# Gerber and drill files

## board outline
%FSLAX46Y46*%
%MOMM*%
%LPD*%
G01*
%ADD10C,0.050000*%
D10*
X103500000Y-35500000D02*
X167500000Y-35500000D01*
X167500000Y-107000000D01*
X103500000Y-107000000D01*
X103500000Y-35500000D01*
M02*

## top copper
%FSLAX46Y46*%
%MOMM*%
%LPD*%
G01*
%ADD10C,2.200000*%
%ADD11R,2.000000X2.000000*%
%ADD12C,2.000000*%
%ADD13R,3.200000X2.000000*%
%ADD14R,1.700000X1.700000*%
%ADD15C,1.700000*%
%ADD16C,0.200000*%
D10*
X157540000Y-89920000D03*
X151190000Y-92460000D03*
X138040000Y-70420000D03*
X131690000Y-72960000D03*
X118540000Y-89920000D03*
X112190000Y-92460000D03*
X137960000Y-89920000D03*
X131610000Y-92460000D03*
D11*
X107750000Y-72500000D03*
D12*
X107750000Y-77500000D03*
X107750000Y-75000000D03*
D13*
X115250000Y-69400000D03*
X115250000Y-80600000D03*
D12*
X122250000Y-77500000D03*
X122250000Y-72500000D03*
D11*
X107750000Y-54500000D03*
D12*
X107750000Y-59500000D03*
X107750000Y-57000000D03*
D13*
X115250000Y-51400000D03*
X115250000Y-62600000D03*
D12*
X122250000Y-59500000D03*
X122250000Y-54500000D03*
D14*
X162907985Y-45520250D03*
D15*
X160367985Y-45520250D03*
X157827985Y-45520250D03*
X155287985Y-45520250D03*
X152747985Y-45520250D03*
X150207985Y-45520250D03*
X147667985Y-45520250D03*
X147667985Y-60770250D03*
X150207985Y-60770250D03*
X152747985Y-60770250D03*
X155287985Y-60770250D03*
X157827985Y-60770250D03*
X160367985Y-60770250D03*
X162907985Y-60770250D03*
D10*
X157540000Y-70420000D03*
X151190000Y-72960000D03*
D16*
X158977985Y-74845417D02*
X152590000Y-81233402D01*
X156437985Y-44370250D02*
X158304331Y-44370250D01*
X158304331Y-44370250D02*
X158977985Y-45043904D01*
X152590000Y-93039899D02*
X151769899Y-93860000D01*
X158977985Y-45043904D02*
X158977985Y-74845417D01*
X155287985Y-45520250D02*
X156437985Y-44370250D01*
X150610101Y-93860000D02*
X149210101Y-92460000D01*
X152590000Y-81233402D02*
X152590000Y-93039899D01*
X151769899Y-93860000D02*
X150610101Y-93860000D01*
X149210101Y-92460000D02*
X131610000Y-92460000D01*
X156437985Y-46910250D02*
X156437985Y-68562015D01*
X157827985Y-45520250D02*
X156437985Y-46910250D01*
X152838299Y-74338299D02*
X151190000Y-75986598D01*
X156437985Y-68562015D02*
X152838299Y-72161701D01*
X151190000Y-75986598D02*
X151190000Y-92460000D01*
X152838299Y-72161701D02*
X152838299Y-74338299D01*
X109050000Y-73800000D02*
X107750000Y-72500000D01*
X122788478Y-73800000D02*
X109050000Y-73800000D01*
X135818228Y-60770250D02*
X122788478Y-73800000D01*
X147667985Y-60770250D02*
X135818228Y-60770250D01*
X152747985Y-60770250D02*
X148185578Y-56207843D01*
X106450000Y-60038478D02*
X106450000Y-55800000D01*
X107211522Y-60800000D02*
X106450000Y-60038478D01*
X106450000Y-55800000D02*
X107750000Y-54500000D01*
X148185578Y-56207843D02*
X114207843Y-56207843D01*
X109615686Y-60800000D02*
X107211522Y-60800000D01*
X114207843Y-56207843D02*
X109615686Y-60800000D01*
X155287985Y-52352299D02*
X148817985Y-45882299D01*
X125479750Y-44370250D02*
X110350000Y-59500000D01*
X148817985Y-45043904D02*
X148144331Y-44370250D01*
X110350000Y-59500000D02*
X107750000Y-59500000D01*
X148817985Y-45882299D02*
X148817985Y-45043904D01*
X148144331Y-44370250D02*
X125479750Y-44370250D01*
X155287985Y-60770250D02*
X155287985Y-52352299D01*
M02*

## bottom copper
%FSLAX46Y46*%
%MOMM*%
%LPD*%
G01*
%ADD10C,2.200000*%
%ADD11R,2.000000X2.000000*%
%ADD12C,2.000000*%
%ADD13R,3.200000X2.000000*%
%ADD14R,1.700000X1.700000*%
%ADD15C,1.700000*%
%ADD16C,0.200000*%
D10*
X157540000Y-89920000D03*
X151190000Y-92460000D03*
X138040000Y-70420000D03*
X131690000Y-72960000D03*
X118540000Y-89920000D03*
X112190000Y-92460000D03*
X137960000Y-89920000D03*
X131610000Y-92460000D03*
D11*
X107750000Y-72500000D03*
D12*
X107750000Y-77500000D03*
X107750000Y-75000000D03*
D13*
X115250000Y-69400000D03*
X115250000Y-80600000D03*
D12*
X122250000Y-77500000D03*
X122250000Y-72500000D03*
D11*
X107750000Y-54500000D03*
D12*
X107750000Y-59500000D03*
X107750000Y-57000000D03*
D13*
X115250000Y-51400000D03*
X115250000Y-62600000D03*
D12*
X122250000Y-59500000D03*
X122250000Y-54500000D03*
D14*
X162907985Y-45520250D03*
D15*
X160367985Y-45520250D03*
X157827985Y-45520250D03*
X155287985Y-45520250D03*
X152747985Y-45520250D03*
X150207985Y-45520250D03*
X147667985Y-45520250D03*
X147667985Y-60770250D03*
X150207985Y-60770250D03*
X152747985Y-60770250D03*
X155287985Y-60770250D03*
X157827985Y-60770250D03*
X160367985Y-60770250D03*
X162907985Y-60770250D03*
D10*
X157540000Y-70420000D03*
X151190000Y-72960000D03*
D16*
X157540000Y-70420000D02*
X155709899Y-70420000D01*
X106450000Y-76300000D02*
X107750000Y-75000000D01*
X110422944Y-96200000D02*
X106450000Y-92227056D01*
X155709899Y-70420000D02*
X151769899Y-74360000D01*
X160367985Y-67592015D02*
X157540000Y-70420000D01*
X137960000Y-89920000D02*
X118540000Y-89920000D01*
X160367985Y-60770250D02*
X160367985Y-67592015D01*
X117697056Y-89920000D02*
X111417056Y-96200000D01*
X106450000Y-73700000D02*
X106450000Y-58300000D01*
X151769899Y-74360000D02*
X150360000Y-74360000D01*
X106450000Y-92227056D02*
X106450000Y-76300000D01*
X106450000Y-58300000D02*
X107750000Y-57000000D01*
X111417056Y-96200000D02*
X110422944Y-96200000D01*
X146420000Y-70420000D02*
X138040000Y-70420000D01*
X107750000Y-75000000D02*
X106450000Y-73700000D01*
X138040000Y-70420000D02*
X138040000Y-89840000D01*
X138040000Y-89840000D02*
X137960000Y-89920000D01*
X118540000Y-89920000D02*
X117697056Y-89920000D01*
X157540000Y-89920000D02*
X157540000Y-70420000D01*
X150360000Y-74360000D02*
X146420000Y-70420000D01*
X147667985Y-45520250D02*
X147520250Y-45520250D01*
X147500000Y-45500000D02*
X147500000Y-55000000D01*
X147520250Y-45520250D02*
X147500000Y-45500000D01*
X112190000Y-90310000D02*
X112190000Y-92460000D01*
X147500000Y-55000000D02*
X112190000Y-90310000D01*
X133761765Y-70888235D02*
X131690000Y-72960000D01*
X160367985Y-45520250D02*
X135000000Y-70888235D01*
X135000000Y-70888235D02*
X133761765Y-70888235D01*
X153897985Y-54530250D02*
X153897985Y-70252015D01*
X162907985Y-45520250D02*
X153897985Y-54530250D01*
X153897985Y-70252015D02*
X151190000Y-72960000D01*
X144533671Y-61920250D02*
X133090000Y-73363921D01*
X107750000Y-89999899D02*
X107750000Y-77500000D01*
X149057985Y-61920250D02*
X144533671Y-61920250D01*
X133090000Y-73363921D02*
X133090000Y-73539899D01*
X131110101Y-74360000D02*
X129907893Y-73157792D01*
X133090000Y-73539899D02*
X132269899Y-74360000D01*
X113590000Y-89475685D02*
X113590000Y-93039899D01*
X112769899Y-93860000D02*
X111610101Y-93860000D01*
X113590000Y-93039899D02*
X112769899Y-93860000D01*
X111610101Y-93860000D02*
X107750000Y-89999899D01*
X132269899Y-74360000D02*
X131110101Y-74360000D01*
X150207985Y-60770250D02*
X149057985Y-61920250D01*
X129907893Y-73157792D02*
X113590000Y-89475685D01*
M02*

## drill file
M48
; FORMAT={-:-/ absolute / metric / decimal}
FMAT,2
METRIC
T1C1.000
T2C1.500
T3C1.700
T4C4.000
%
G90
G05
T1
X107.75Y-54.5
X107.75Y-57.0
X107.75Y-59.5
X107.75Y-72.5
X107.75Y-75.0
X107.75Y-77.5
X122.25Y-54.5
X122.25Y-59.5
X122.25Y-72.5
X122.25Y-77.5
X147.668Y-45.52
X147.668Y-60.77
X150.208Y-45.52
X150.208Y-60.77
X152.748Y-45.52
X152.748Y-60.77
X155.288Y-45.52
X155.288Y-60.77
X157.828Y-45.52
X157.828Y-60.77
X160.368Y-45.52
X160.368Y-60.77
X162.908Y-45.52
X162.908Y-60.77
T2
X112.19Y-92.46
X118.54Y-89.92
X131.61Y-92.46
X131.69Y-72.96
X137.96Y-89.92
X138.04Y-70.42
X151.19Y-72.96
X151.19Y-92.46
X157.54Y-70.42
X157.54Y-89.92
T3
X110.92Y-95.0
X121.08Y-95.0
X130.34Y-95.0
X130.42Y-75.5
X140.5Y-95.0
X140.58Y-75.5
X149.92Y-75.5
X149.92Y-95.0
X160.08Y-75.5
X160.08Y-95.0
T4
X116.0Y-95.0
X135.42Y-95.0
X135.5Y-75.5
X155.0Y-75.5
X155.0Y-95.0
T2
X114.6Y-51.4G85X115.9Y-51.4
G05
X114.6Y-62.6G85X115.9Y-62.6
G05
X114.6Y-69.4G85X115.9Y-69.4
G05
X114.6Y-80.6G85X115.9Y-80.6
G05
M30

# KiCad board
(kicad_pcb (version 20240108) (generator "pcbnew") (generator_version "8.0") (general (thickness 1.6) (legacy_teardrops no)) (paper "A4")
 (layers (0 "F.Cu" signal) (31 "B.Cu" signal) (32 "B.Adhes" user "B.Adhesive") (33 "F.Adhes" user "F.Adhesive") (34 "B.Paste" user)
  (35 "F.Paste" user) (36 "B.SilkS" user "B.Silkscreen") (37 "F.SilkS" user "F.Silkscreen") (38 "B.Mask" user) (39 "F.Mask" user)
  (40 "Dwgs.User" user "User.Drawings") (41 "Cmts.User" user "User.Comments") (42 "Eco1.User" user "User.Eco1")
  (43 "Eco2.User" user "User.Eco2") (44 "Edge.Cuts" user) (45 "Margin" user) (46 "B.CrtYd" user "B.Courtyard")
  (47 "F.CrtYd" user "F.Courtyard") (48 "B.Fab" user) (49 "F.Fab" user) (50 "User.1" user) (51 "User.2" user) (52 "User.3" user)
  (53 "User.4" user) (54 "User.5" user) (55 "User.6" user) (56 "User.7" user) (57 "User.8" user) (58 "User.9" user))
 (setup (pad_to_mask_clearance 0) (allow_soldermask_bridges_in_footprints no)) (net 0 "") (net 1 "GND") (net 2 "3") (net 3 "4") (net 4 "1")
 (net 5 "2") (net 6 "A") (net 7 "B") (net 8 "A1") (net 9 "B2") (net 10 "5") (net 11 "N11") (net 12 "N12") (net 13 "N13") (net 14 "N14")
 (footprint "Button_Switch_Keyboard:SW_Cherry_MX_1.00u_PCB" (layer "F.Cu") (at 157.54 89.92)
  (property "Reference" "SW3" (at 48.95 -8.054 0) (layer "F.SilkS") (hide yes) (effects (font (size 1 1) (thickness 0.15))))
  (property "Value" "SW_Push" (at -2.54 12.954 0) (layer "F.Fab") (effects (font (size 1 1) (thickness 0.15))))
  (pad "" np_thru_hole circle (at -7.62 5.08) (size 1.7 1.7) (drill 1.7) (layers "*.Cu" "*.Mask"))
  (pad "" np_thru_hole circle (at -2.54 5.08) (size 4 4) (drill 4) (layers "*.Cu" "*.Mask"))
  (pad "" np_thru_hole circle (at 2.54 5.08) (size 1.7 1.7) (drill 1.7) (layers "*.Cu" "*.Mask"))
  (pad "1" thru_hole circle (at 0 0) (size 2.2 2.2) (drill 1.5) (layers "*.Cu" "*.Mask") (remove_unused_layers no) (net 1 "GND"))
  (pad "2" thru_hole circle (at -6.35 2.54) (size 2.2 2.2) (drill 1.5) (layers "*.Cu" "*.Mask") (remove_unused_layers no) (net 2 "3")))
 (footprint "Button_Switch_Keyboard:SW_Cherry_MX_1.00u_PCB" (layer "F.Cu") (at 138.04 70.42)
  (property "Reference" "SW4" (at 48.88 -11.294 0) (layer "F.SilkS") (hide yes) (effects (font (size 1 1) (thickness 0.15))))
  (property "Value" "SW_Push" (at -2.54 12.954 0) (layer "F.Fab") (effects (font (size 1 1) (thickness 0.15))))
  (pad "" np_thru_hole circle (at -7.62 5.08) (size 1.7 1.7) (drill 1.7) (layers "*.Cu" "*.Mask"))
  (pad "" np_thru_hole circle (at -2.54 5.08) (size 4 4) (drill 4) (layers "*.Cu" "*.Mask"))
  (pad "" np_thru_hole circle (at 2.54 5.08) (size 1.7 1.7) (drill 1.7) (layers "*.Cu" "*.Mask"))
  (pad "1" thru_hole circle (at 0 0) (size 2.2 2.2) (drill 1.5) (layers "*.Cu" "*.Mask") (remove_unused_layers no) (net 1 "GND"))
  (pad "2" thru_hole circle (at -6.35 2.54) (size 2.2 2.2) (drill 1.5) (layers "*.Cu" "*.Mask") (remove_unused_layers no) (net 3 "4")))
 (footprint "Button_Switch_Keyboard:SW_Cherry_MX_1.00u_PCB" (layer "F.Cu") (at 118.54 89.92)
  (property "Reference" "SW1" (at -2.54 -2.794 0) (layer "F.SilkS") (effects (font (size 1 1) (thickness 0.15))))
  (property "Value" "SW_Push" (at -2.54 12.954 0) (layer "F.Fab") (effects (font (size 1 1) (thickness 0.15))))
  (pad "" np_thru_hole circle (at -7.62 5.08) (size 1.7 1.7) (drill 1.7) (layers "*.Cu" "*.Mask"))
  (pad "" np_thru_hole circle (at -2.54 5.08) (size 4 4) (drill 4) (layers "*.Cu" "*.Mask"))
  (pad "" np_thru_hole circle (at 2.54 5.08) (size 1.7 1.7) (drill 1.7) (layers "*.Cu" "*.Mask"))
  (pad "1" thru_hole circle (at 0 0) (size 2.2 2.2) (drill 1.5) (layers "*.Cu" "*.Mask") (remove_unused_layers no) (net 1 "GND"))
  (pad "2" thru_hole circle (at -6.35 2.54) (size 2.2 2.2) (drill 1.5) (layers "*.Cu" "*.Mask") (remove_unused_layers no) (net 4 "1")))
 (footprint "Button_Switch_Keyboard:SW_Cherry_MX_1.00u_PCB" (layer "F.Cu") (at 137.96 89.92)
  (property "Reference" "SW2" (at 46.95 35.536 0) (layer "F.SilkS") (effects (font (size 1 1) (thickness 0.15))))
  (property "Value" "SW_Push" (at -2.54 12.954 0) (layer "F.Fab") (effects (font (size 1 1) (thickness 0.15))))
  (pad "" np_thru_hole circle (at -7.62 5.08) (size 1.7 1.7) (drill 1.7) (layers "*.Cu" "*.Mask"))
  (pad "" np_thru_hole circle (at -2.54 5.08) (size 4 4) (drill 4) (layers "*.Cu" "*.Mask"))
  (pad "" np_thru_hole circle (at 2.54 5.08) (size 1.7 1.7) (drill 1.7) (layers "*.Cu" "*.Mask"))
  (pad "1" thru_hole circle (at 0 0) (size 2.2 2.2) (drill 1.5) (layers "*.Cu" "*.Mask") (remove_unused_layers no) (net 1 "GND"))
  (pad "2" thru_hole circle (at -6.35 2.54) (size 2.2 2.2) (drill 1.5) (layers "*.Cu" "*.Mask") (remove_unused_layers no) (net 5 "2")))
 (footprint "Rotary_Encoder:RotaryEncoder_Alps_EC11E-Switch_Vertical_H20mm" (layer "F.Cu") (at 107.75 72.5)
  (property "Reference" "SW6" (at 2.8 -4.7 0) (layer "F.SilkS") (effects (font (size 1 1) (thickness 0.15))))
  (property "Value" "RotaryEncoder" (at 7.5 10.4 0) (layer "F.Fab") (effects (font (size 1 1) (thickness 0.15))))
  (pad "A" thru_hole rect (at 0 0) (size 2 2) (drill 1) (layers "*.Cu" "*.Mask") (remove_unused_layers no) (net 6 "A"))
  (pad "B" thru_hole circle (at 0 5) (size 2 2) (drill 1) (layers "*.Cu" "*.Mask") (remove_unused_layers no) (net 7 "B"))
  (pad "C" thru_hole circle (at 0 2.5) (size 2 2) (drill 1) (layers "*.Cu" "*.Mask") (remove_unused_layers no) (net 1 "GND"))
  (pad "MP" thru_hole rect (at 7.5 -3.1) (size 3.2 2) (drill oval 2.8 1.5) (layers "*.Cu" "*.Mask") (remove_unused_layers no))
  (pad "MP" thru_hole rect (at 7.5 8.1) (size 3.2 2) (drill oval 2.8 1.5) (layers "*.Cu" "*.Mask") (remove_unused_layers no))
  (pad "S1" thru_hole circle (at 14.5 5) (size 2 2) (drill 1) (layers "*.Cu" "*.Mask") (remove_unused_layers no))
  (pad "S2" thru_hole circle (at 14.5 0) (size 2 2) (drill 1) (layers "*.Cu" "*.Mask") (remove_unused_layers no)))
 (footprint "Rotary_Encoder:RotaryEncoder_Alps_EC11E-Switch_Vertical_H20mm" (layer "F.Cu") (at 107.75 54.5)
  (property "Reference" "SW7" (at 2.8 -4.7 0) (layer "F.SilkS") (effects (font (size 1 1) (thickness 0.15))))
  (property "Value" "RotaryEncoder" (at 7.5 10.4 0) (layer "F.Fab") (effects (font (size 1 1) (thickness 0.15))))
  (pad "A" thru_hole rect (at 0 0) (size 2 2) (drill 1) (layers "*.Cu" "*.Mask") (remove_unused_layers no) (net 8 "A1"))
  (pad "B" thru_hole circle (at 0 5) (size 2 2) (drill 1) (layers "*.Cu" "*.Mask") (remove_unused_layers no) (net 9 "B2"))
  (pad "C" thru_hole circle (at 0 2.5) (size 2 2) (drill 1) (layers "*.Cu" "*.Mask") (remove_unused_layers no) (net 1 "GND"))
  (pad "MP" thru_hole rect (at 7.5 -3.1) (size 3.2 2) (drill oval 2.8 1.5) (layers "*.Cu" "*.Mask") (remove_unused_layers no))
  (pad "MP" thru_hole rect (at 7.5 8.1) (size 3.2 2) (drill oval 2.8 1.5) (layers "*.Cu" "*.Mask") (remove_unused_layers no))
  (pad "S1" thru_hole circle (at 14.5 5) (size 2 2) (drill 1) (layers "*.Cu" "*.Mask") (remove_unused_layers no))
  (pad "S2" thru_hole circle (at 14.5 0) (size 2 2) (drill 1) (layers "*.Cu" "*.Mask") (remove_unused_layers no)))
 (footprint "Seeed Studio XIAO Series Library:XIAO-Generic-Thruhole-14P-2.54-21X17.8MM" (layer "F.Cu") (at 155.287985 53.14525 -90)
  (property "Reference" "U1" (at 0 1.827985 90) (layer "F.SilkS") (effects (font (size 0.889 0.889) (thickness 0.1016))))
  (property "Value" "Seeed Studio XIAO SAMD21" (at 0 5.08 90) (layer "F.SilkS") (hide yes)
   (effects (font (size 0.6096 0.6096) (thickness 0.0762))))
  (pad "1" thru_hole rect (at -7.625 -7.62 270) (size 1.7 1.7) (drill 1) (layers "*.Cu" "*.Mask") (remove_unused_layers no) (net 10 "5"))
  (pad "2" thru_hole circle (at -7.625 -5.08 270) (size 1.7 1.7) (drill 1) (layers "*.Cu" "*.Mask") (remove_unused_layers no) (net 3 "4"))
  (pad "3" thru_hole circle (at -7.625 -2.54 270) (size 1.7 1.7) (drill 1) (layers "*.Cu" "*.Mask") (remove_unused_layers no) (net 2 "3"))
  (pad "4" thru_hole circle (at -7.625 0 270) (size 1.7 1.7) (drill 1) (layers "*.Cu" "*.Mask") (remove_unused_layers no) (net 5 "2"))
  (pad "5" thru_hole circle (at -7.625 2.54 270) (size 1.7 1.7) (drill 1) (layers "*.Cu" "*.Mask") (remove_unused_layers no) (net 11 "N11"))
  (pad "6" thru_hole circle (at -7.625 5.08 90) (size 1.7 1.7) (drill 1) (layers "*.Cu" "*.Mask") (remove_unused_layers no) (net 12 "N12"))
  (pad "7" thru_hole circle (at -7.625 7.62 270) (size 1.7 1.7) (drill 1) (layers "*.Cu" "*.Mask") (remove_unused_layers no) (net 4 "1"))
  (pad "8" thru_hole circle (at 7.625 7.62 270) (size 1.7 1.7) (drill 1) (layers "*.Cu" "*.Mask") (remove_unused_layers no) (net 6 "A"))
  (pad "9" thru_hole circle (at 7.625 5.08 270) (size 1.7 1.7) (drill 1) (layers "*.Cu" "*.Mask") (remove_unused_layers no) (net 7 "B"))
  (pad "10" thru_hole circle (at 7.625 2.54 270) (size 1.7 1.7) (drill 1) (layers "*.Cu" "*.Mask") (remove_unused_layers no) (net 8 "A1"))
  (pad "11" thru_hole circle (at 7.625 0 270) (size 1.7 1.7) (drill 1) (layers "*.Cu" "*.Mask") (remove_unused_layers no) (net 9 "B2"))
  (pad "12" thru_hole circle (at 7.625 -2.54 270) (size 1.7 1.7) (drill 1) (layers "*.Cu" "*.Mask") (remove_unused_layers no) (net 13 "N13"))
  (pad "13" thru_hole circle (at 7.625 -5.08 270) (size 1.7 1.7) (drill 1) (layers "*.Cu" "*.Mask") (remove_unused_layers no) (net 1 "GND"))
  (pad "14" thru_hole circle (at 7.625 -7.62 270) (size 1.7 1.7) (drill 1) (layers "*.Cu" "*.Mask") (remove_unused_layers no) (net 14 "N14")))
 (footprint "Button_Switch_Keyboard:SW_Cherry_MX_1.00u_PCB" (layer "F.Cu") (at 157.54 70.42)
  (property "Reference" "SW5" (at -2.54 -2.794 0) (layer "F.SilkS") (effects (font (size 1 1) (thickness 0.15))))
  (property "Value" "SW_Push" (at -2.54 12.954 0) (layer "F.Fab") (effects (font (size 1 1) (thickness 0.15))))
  (pad "" np_thru_hole circle (at -7.62 5.08) (size 1.7 1.7) (drill 1.7) (layers "*.Cu" "*.Mask"))
  (pad "" np_thru_hole circle (at -2.54 5.08) (size 4 4) (drill 4) (layers "*.Cu" "*.Mask"))
  (pad "" np_thru_hole circle (at 2.54 5.08) (size 1.7 1.7) (drill 1.7) (layers "*.Cu" "*.Mask"))
  (pad "1" thru_hole circle (at 0 0) (size 2.2 2.2) (drill 1.5) (layers "*.Cu" "*.Mask") (remove_unused_layers no) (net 1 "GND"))
  (pad "2" thru_hole circle (at -6.35 2.54) (size 2.2 2.2) (drill 1.5) (layers "*.Cu" "*.Mask") (remove_unused_layers no) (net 10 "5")))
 (gr_rect (start 103.5 35.5) (end 167.5 107) (stroke (width 0.05) (type default)) (fill none) (layer "Edge.Cuts"))
 (segment (start 157.54 70.42) (end 155.709899 70.42) (width 0.2) (layer "B.Cu") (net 1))
 (segment (start 106.45 76.3) (end 107.75 75) (width 0.2) (layer "B.Cu") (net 1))
 (segment (start 110.422944 96.2) (end 106.45 92.227056) (width 0.2) (layer "B.Cu") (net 1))
 (segment (start 155.709899 70.42) (end 151.769899 74.36) (width 0.2) (layer "B.Cu") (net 1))
 (segment (start 160.367985 67.592015) (end 157.54 70.42) (width 0.2) (layer "B.Cu") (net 1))
 (segment (start 137.96 89.92) (end 118.54 89.92) (width 0.2) (layer "B.Cu") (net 1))
 (segment (start 160.367985 60.77025) (end 160.367985 67.592015) (width 0.2) (layer "B.Cu") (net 1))
 (segment (start 117.697056 89.92) (end 111.417056 96.2) (width 0.2) (layer "B.Cu") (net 1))
 (segment (start 106.45 73.7) (end 106.45 58.3) (width 0.2) (layer "B.Cu") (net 1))
 (segment (start 151.769899 74.36) (end 150.36 74.36) (width 0.2) (layer "B.Cu") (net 1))
 (segment (start 106.45 92.227056) (end 106.45 76.3) (width 0.2) (layer "B.Cu") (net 1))
 (segment (start 106.45 58.3) (end 107.75 57) (width 0.2) (layer "B.Cu") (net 1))
 (segment (start 111.417056 96.2) (end 110.422944 96.2) (width 0.2) (layer "B.Cu") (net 1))
 (segment (start 146.42 70.42) (end 138.04 70.42) (width 0.2) (layer "B.Cu") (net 1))
 (segment (start 107.75 75) (end 106.45 73.7) (width 0.2) (layer "B.Cu") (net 1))
 (segment (start 138.04 70.42) (end 138.04 89.84) (width 0.2) (layer "B.Cu") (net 1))
 (segment (start 138.04 89.84) (end 137.96 89.92) (width 0.2) (layer "B.Cu") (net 1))
 (segment (start 118.54 89.92) (end 117.697056 89.92) (width 0.2) (layer "B.Cu") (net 1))
 (segment (start 157.54 89.92) (end 157.54 70.42) (width 0.2) (layer "B.Cu") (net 1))
 (segment (start 150.36 74.36) (end 146.42 70.42) (width 0.2) (layer "B.Cu") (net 1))
 (segment (start 147.667985 45.52025) (end 147.52025 45.52025) (width 0.2) (layer "B.Cu") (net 4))
 (segment (start 147.5 45.5) (end 147.5 55) (width 0.2) (layer "B.Cu") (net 4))
 (segment (start 147.52025 45.52025) (end 147.5 45.5) (width 0.2) (layer "B.Cu") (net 4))
 (segment (start 112.19 90.31) (end 112.19 92.46) (width 0.2) (layer "B.Cu") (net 4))
 (segment (start 147.5 55) (end 112.19 90.31) (width 0.2) (layer "B.Cu") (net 4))
 (segment (start 158.977985 74.845417) (end 152.59 81.233402) (width 0.2) (layer "F.Cu") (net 5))
 (segment (start 156.437985 44.37025) (end 158.304331 44.37025) (width 0.2) (layer "F.Cu") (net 5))
 (segment (start 158.304331 44.37025) (end 158.977985 45.043904) (width 0.2) (layer "F.Cu") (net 5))
 (segment (start 152.59 93.039899) (end 151.769899 93.86) (width 0.2) (layer "F.Cu") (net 5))
 (segment (start 158.977985 45.043904) (end 158.977985 74.845417) (width 0.2) (layer "F.Cu") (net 5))
 (segment (start 155.287985 45.52025) (end 156.437985 44.37025) (width 0.2) (layer "F.Cu") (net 5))
 (segment (start 150.610101 93.86) (end 149.210101 92.46) (width 0.2) (layer "F.Cu") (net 5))
 (segment (start 152.59 81.233402) (end 152.59 93.039899) (width 0.2) (layer "F.Cu") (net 5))
 (segment (start 151.769899 93.86) (end 150.610101 93.86) (width 0.2) (layer "F.Cu") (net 5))
 (segment (start 149.210101 92.46) (end 131.61 92.46) (width 0.2) (layer "F.Cu") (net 5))
 (segment (start 156.437985 46.91025) (end 156.437985 68.562015) (width 0.2) (layer "F.Cu") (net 2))
 (segment (start 157.827985 45.52025) (end 156.437985 46.91025) (width 0.2) (layer "F.Cu") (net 2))
 (segment (start 152.838299 74.338299) (end 151.19 75.986598) (width 0.2) (layer "F.Cu") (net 2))
 (segment (start 156.437985 68.562015) (end 152.838299 72.161701) (width 0.2) (layer "F.Cu") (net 2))
 (segment (start 151.19 75.986598) (end 151.19 92.46) (width 0.2) (layer "F.Cu") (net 2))
 (segment (start 152.838299 72.161701) (end 152.838299 74.338299) (width 0.2) (layer "F.Cu") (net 2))
 (segment (start 133.761765 70.888235) (end 131.69 72.96) (width 0.2) (layer "B.Cu") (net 3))
 (segment (start 160.367985 45.52025) (end 135 70.888235) (width 0.2) (layer "B.Cu") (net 3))
 (segment (start 135 70.888235) (end 133.761765 70.888235) (width 0.2) (layer "B.Cu") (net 3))
 (segment (start 153.897985 54.53025) (end 153.897985 70.252015) (width 0.2) (layer "B.Cu") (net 10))
 (segment (start 162.907985 45.52025) (end 153.897985 54.53025) (width 0.2) (layer "B.Cu") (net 10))
 (segment (start 153.897985 70.252015) (end 151.19 72.96) (width 0.2) (layer "B.Cu") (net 10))
 (segment (start 144.533671 61.92025) (end 133.09 73.363921) (width 0.2) (layer "B.Cu") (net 7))
 (segment (start 107.75 89.999899) (end 107.75 77.5) (width 0.2) (layer "B.Cu") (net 7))
 (segment (start 149.057985 61.92025) (end 144.533671 61.92025) (width 0.2) (layer "B.Cu") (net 7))
 (segment (start 133.09 73.363921) (end 133.09 73.539899) (width 0.2) (layer "B.Cu") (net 7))
 (segment (start 131.110101 74.36) (end 129.907893 73.157792) (width 0.2) (layer "B.Cu") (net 7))
 (segment (start 133.09 73.539899) (end 132.269899 74.36) (width 0.2) (layer "B.Cu") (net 7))
 (segment (start 113.59 89.475685) (end 113.59 93.039899) (width 0.2) (layer "B.Cu") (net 7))
 (segment (start 112.769899 93.86) (end 111.610101 93.86) (width 0.2) (layer "B.Cu") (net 7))
 (segment (start 113.59 93.039899) (end 112.769899 93.86) (width 0.2) (layer "B.Cu") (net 7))
 (segment (start 111.610101 93.86) (end 107.75 89.999899) (width 0.2) (layer "B.Cu") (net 7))
 (segment (start 132.269899 74.36) (end 131.110101 74.36) (width 0.2) (layer "B.Cu") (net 7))
 (segment (start 150.207985 60.77025) (end 149.057985 61.92025) (width 0.2) (layer "B.Cu") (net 7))
 (segment (start 129.907893 73.157792) (end 113.59 89.475685) (width 0.2) (layer "B.Cu") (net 7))
 (segment (start 109.05 73.8) (end 107.75 72.5) (width 0.2) (layer "F.Cu") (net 6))
 (segment (start 122.788478 73.8) (end 109.05 73.8) (width 0.2) (layer "F.Cu") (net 6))
 (segment (start 135.818228 60.77025) (end 122.788478 73.8) (width 0.2) (layer "F.Cu") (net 6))
 (segment (start 147.667985 60.77025) (end 135.818228 60.77025) (width 0.2) (layer "F.Cu") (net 6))
 (segment (start 152.747985 60.77025) (end 148.185578 56.207843) (width 0.2) (layer "F.Cu") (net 8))
 (segment (start 106.45 60.038478) (end 106.45 55.8) (width 0.2) (layer "F.Cu") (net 8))
 (segment (start 107.211522 60.8) (end 106.45 60.038478) (width 0.2) (layer "F.Cu") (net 8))
 (segment (start 106.45 55.8) (end 107.75 54.5) (width 0.2) (layer "F.Cu") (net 8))
 (segment (start 148.185578 56.207843) (end 114.207843 56.207843) (width 0.2) (layer "F.Cu") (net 8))
 (segment (start 109.615686 60.8) (end 107.211522 60.8) (width 0.2) (layer "F.Cu") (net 8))
 (segment (start 114.207843 56.207843) (end 109.615686 60.8) (width 0.2) (layer "F.Cu") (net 8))
 (segment (start 155.287985 52.352299) (end 148.817985 45.882299) (width 0.2) (layer "F.Cu") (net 9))
 (segment (start 125.47975 44.37025) (end 110.35 59.5) (width 0.2) (layer "F.Cu") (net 9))
 (segment (start 148.817985 45.043904) (end 148.144331 44.37025) (width 0.2) (layer "F.Cu") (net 9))
 (segment (start 110.35 59.5) (end 107.75 59.5) (width 0.2) (layer "F.Cu") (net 9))
 (segment (start 148.817985 45.882299) (end 148.817985 45.043904) (width 0.2) (layer "F.Cu") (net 9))
 (segment (start 148.144331 44.37025) (end 125.47975 44.37025) (width 0.2) (layer "F.Cu") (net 9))
 (segment (start 155.287985 60.77025) (end 155.287985 52.352299) (width 0.2) (layer "F.Cu") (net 9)))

